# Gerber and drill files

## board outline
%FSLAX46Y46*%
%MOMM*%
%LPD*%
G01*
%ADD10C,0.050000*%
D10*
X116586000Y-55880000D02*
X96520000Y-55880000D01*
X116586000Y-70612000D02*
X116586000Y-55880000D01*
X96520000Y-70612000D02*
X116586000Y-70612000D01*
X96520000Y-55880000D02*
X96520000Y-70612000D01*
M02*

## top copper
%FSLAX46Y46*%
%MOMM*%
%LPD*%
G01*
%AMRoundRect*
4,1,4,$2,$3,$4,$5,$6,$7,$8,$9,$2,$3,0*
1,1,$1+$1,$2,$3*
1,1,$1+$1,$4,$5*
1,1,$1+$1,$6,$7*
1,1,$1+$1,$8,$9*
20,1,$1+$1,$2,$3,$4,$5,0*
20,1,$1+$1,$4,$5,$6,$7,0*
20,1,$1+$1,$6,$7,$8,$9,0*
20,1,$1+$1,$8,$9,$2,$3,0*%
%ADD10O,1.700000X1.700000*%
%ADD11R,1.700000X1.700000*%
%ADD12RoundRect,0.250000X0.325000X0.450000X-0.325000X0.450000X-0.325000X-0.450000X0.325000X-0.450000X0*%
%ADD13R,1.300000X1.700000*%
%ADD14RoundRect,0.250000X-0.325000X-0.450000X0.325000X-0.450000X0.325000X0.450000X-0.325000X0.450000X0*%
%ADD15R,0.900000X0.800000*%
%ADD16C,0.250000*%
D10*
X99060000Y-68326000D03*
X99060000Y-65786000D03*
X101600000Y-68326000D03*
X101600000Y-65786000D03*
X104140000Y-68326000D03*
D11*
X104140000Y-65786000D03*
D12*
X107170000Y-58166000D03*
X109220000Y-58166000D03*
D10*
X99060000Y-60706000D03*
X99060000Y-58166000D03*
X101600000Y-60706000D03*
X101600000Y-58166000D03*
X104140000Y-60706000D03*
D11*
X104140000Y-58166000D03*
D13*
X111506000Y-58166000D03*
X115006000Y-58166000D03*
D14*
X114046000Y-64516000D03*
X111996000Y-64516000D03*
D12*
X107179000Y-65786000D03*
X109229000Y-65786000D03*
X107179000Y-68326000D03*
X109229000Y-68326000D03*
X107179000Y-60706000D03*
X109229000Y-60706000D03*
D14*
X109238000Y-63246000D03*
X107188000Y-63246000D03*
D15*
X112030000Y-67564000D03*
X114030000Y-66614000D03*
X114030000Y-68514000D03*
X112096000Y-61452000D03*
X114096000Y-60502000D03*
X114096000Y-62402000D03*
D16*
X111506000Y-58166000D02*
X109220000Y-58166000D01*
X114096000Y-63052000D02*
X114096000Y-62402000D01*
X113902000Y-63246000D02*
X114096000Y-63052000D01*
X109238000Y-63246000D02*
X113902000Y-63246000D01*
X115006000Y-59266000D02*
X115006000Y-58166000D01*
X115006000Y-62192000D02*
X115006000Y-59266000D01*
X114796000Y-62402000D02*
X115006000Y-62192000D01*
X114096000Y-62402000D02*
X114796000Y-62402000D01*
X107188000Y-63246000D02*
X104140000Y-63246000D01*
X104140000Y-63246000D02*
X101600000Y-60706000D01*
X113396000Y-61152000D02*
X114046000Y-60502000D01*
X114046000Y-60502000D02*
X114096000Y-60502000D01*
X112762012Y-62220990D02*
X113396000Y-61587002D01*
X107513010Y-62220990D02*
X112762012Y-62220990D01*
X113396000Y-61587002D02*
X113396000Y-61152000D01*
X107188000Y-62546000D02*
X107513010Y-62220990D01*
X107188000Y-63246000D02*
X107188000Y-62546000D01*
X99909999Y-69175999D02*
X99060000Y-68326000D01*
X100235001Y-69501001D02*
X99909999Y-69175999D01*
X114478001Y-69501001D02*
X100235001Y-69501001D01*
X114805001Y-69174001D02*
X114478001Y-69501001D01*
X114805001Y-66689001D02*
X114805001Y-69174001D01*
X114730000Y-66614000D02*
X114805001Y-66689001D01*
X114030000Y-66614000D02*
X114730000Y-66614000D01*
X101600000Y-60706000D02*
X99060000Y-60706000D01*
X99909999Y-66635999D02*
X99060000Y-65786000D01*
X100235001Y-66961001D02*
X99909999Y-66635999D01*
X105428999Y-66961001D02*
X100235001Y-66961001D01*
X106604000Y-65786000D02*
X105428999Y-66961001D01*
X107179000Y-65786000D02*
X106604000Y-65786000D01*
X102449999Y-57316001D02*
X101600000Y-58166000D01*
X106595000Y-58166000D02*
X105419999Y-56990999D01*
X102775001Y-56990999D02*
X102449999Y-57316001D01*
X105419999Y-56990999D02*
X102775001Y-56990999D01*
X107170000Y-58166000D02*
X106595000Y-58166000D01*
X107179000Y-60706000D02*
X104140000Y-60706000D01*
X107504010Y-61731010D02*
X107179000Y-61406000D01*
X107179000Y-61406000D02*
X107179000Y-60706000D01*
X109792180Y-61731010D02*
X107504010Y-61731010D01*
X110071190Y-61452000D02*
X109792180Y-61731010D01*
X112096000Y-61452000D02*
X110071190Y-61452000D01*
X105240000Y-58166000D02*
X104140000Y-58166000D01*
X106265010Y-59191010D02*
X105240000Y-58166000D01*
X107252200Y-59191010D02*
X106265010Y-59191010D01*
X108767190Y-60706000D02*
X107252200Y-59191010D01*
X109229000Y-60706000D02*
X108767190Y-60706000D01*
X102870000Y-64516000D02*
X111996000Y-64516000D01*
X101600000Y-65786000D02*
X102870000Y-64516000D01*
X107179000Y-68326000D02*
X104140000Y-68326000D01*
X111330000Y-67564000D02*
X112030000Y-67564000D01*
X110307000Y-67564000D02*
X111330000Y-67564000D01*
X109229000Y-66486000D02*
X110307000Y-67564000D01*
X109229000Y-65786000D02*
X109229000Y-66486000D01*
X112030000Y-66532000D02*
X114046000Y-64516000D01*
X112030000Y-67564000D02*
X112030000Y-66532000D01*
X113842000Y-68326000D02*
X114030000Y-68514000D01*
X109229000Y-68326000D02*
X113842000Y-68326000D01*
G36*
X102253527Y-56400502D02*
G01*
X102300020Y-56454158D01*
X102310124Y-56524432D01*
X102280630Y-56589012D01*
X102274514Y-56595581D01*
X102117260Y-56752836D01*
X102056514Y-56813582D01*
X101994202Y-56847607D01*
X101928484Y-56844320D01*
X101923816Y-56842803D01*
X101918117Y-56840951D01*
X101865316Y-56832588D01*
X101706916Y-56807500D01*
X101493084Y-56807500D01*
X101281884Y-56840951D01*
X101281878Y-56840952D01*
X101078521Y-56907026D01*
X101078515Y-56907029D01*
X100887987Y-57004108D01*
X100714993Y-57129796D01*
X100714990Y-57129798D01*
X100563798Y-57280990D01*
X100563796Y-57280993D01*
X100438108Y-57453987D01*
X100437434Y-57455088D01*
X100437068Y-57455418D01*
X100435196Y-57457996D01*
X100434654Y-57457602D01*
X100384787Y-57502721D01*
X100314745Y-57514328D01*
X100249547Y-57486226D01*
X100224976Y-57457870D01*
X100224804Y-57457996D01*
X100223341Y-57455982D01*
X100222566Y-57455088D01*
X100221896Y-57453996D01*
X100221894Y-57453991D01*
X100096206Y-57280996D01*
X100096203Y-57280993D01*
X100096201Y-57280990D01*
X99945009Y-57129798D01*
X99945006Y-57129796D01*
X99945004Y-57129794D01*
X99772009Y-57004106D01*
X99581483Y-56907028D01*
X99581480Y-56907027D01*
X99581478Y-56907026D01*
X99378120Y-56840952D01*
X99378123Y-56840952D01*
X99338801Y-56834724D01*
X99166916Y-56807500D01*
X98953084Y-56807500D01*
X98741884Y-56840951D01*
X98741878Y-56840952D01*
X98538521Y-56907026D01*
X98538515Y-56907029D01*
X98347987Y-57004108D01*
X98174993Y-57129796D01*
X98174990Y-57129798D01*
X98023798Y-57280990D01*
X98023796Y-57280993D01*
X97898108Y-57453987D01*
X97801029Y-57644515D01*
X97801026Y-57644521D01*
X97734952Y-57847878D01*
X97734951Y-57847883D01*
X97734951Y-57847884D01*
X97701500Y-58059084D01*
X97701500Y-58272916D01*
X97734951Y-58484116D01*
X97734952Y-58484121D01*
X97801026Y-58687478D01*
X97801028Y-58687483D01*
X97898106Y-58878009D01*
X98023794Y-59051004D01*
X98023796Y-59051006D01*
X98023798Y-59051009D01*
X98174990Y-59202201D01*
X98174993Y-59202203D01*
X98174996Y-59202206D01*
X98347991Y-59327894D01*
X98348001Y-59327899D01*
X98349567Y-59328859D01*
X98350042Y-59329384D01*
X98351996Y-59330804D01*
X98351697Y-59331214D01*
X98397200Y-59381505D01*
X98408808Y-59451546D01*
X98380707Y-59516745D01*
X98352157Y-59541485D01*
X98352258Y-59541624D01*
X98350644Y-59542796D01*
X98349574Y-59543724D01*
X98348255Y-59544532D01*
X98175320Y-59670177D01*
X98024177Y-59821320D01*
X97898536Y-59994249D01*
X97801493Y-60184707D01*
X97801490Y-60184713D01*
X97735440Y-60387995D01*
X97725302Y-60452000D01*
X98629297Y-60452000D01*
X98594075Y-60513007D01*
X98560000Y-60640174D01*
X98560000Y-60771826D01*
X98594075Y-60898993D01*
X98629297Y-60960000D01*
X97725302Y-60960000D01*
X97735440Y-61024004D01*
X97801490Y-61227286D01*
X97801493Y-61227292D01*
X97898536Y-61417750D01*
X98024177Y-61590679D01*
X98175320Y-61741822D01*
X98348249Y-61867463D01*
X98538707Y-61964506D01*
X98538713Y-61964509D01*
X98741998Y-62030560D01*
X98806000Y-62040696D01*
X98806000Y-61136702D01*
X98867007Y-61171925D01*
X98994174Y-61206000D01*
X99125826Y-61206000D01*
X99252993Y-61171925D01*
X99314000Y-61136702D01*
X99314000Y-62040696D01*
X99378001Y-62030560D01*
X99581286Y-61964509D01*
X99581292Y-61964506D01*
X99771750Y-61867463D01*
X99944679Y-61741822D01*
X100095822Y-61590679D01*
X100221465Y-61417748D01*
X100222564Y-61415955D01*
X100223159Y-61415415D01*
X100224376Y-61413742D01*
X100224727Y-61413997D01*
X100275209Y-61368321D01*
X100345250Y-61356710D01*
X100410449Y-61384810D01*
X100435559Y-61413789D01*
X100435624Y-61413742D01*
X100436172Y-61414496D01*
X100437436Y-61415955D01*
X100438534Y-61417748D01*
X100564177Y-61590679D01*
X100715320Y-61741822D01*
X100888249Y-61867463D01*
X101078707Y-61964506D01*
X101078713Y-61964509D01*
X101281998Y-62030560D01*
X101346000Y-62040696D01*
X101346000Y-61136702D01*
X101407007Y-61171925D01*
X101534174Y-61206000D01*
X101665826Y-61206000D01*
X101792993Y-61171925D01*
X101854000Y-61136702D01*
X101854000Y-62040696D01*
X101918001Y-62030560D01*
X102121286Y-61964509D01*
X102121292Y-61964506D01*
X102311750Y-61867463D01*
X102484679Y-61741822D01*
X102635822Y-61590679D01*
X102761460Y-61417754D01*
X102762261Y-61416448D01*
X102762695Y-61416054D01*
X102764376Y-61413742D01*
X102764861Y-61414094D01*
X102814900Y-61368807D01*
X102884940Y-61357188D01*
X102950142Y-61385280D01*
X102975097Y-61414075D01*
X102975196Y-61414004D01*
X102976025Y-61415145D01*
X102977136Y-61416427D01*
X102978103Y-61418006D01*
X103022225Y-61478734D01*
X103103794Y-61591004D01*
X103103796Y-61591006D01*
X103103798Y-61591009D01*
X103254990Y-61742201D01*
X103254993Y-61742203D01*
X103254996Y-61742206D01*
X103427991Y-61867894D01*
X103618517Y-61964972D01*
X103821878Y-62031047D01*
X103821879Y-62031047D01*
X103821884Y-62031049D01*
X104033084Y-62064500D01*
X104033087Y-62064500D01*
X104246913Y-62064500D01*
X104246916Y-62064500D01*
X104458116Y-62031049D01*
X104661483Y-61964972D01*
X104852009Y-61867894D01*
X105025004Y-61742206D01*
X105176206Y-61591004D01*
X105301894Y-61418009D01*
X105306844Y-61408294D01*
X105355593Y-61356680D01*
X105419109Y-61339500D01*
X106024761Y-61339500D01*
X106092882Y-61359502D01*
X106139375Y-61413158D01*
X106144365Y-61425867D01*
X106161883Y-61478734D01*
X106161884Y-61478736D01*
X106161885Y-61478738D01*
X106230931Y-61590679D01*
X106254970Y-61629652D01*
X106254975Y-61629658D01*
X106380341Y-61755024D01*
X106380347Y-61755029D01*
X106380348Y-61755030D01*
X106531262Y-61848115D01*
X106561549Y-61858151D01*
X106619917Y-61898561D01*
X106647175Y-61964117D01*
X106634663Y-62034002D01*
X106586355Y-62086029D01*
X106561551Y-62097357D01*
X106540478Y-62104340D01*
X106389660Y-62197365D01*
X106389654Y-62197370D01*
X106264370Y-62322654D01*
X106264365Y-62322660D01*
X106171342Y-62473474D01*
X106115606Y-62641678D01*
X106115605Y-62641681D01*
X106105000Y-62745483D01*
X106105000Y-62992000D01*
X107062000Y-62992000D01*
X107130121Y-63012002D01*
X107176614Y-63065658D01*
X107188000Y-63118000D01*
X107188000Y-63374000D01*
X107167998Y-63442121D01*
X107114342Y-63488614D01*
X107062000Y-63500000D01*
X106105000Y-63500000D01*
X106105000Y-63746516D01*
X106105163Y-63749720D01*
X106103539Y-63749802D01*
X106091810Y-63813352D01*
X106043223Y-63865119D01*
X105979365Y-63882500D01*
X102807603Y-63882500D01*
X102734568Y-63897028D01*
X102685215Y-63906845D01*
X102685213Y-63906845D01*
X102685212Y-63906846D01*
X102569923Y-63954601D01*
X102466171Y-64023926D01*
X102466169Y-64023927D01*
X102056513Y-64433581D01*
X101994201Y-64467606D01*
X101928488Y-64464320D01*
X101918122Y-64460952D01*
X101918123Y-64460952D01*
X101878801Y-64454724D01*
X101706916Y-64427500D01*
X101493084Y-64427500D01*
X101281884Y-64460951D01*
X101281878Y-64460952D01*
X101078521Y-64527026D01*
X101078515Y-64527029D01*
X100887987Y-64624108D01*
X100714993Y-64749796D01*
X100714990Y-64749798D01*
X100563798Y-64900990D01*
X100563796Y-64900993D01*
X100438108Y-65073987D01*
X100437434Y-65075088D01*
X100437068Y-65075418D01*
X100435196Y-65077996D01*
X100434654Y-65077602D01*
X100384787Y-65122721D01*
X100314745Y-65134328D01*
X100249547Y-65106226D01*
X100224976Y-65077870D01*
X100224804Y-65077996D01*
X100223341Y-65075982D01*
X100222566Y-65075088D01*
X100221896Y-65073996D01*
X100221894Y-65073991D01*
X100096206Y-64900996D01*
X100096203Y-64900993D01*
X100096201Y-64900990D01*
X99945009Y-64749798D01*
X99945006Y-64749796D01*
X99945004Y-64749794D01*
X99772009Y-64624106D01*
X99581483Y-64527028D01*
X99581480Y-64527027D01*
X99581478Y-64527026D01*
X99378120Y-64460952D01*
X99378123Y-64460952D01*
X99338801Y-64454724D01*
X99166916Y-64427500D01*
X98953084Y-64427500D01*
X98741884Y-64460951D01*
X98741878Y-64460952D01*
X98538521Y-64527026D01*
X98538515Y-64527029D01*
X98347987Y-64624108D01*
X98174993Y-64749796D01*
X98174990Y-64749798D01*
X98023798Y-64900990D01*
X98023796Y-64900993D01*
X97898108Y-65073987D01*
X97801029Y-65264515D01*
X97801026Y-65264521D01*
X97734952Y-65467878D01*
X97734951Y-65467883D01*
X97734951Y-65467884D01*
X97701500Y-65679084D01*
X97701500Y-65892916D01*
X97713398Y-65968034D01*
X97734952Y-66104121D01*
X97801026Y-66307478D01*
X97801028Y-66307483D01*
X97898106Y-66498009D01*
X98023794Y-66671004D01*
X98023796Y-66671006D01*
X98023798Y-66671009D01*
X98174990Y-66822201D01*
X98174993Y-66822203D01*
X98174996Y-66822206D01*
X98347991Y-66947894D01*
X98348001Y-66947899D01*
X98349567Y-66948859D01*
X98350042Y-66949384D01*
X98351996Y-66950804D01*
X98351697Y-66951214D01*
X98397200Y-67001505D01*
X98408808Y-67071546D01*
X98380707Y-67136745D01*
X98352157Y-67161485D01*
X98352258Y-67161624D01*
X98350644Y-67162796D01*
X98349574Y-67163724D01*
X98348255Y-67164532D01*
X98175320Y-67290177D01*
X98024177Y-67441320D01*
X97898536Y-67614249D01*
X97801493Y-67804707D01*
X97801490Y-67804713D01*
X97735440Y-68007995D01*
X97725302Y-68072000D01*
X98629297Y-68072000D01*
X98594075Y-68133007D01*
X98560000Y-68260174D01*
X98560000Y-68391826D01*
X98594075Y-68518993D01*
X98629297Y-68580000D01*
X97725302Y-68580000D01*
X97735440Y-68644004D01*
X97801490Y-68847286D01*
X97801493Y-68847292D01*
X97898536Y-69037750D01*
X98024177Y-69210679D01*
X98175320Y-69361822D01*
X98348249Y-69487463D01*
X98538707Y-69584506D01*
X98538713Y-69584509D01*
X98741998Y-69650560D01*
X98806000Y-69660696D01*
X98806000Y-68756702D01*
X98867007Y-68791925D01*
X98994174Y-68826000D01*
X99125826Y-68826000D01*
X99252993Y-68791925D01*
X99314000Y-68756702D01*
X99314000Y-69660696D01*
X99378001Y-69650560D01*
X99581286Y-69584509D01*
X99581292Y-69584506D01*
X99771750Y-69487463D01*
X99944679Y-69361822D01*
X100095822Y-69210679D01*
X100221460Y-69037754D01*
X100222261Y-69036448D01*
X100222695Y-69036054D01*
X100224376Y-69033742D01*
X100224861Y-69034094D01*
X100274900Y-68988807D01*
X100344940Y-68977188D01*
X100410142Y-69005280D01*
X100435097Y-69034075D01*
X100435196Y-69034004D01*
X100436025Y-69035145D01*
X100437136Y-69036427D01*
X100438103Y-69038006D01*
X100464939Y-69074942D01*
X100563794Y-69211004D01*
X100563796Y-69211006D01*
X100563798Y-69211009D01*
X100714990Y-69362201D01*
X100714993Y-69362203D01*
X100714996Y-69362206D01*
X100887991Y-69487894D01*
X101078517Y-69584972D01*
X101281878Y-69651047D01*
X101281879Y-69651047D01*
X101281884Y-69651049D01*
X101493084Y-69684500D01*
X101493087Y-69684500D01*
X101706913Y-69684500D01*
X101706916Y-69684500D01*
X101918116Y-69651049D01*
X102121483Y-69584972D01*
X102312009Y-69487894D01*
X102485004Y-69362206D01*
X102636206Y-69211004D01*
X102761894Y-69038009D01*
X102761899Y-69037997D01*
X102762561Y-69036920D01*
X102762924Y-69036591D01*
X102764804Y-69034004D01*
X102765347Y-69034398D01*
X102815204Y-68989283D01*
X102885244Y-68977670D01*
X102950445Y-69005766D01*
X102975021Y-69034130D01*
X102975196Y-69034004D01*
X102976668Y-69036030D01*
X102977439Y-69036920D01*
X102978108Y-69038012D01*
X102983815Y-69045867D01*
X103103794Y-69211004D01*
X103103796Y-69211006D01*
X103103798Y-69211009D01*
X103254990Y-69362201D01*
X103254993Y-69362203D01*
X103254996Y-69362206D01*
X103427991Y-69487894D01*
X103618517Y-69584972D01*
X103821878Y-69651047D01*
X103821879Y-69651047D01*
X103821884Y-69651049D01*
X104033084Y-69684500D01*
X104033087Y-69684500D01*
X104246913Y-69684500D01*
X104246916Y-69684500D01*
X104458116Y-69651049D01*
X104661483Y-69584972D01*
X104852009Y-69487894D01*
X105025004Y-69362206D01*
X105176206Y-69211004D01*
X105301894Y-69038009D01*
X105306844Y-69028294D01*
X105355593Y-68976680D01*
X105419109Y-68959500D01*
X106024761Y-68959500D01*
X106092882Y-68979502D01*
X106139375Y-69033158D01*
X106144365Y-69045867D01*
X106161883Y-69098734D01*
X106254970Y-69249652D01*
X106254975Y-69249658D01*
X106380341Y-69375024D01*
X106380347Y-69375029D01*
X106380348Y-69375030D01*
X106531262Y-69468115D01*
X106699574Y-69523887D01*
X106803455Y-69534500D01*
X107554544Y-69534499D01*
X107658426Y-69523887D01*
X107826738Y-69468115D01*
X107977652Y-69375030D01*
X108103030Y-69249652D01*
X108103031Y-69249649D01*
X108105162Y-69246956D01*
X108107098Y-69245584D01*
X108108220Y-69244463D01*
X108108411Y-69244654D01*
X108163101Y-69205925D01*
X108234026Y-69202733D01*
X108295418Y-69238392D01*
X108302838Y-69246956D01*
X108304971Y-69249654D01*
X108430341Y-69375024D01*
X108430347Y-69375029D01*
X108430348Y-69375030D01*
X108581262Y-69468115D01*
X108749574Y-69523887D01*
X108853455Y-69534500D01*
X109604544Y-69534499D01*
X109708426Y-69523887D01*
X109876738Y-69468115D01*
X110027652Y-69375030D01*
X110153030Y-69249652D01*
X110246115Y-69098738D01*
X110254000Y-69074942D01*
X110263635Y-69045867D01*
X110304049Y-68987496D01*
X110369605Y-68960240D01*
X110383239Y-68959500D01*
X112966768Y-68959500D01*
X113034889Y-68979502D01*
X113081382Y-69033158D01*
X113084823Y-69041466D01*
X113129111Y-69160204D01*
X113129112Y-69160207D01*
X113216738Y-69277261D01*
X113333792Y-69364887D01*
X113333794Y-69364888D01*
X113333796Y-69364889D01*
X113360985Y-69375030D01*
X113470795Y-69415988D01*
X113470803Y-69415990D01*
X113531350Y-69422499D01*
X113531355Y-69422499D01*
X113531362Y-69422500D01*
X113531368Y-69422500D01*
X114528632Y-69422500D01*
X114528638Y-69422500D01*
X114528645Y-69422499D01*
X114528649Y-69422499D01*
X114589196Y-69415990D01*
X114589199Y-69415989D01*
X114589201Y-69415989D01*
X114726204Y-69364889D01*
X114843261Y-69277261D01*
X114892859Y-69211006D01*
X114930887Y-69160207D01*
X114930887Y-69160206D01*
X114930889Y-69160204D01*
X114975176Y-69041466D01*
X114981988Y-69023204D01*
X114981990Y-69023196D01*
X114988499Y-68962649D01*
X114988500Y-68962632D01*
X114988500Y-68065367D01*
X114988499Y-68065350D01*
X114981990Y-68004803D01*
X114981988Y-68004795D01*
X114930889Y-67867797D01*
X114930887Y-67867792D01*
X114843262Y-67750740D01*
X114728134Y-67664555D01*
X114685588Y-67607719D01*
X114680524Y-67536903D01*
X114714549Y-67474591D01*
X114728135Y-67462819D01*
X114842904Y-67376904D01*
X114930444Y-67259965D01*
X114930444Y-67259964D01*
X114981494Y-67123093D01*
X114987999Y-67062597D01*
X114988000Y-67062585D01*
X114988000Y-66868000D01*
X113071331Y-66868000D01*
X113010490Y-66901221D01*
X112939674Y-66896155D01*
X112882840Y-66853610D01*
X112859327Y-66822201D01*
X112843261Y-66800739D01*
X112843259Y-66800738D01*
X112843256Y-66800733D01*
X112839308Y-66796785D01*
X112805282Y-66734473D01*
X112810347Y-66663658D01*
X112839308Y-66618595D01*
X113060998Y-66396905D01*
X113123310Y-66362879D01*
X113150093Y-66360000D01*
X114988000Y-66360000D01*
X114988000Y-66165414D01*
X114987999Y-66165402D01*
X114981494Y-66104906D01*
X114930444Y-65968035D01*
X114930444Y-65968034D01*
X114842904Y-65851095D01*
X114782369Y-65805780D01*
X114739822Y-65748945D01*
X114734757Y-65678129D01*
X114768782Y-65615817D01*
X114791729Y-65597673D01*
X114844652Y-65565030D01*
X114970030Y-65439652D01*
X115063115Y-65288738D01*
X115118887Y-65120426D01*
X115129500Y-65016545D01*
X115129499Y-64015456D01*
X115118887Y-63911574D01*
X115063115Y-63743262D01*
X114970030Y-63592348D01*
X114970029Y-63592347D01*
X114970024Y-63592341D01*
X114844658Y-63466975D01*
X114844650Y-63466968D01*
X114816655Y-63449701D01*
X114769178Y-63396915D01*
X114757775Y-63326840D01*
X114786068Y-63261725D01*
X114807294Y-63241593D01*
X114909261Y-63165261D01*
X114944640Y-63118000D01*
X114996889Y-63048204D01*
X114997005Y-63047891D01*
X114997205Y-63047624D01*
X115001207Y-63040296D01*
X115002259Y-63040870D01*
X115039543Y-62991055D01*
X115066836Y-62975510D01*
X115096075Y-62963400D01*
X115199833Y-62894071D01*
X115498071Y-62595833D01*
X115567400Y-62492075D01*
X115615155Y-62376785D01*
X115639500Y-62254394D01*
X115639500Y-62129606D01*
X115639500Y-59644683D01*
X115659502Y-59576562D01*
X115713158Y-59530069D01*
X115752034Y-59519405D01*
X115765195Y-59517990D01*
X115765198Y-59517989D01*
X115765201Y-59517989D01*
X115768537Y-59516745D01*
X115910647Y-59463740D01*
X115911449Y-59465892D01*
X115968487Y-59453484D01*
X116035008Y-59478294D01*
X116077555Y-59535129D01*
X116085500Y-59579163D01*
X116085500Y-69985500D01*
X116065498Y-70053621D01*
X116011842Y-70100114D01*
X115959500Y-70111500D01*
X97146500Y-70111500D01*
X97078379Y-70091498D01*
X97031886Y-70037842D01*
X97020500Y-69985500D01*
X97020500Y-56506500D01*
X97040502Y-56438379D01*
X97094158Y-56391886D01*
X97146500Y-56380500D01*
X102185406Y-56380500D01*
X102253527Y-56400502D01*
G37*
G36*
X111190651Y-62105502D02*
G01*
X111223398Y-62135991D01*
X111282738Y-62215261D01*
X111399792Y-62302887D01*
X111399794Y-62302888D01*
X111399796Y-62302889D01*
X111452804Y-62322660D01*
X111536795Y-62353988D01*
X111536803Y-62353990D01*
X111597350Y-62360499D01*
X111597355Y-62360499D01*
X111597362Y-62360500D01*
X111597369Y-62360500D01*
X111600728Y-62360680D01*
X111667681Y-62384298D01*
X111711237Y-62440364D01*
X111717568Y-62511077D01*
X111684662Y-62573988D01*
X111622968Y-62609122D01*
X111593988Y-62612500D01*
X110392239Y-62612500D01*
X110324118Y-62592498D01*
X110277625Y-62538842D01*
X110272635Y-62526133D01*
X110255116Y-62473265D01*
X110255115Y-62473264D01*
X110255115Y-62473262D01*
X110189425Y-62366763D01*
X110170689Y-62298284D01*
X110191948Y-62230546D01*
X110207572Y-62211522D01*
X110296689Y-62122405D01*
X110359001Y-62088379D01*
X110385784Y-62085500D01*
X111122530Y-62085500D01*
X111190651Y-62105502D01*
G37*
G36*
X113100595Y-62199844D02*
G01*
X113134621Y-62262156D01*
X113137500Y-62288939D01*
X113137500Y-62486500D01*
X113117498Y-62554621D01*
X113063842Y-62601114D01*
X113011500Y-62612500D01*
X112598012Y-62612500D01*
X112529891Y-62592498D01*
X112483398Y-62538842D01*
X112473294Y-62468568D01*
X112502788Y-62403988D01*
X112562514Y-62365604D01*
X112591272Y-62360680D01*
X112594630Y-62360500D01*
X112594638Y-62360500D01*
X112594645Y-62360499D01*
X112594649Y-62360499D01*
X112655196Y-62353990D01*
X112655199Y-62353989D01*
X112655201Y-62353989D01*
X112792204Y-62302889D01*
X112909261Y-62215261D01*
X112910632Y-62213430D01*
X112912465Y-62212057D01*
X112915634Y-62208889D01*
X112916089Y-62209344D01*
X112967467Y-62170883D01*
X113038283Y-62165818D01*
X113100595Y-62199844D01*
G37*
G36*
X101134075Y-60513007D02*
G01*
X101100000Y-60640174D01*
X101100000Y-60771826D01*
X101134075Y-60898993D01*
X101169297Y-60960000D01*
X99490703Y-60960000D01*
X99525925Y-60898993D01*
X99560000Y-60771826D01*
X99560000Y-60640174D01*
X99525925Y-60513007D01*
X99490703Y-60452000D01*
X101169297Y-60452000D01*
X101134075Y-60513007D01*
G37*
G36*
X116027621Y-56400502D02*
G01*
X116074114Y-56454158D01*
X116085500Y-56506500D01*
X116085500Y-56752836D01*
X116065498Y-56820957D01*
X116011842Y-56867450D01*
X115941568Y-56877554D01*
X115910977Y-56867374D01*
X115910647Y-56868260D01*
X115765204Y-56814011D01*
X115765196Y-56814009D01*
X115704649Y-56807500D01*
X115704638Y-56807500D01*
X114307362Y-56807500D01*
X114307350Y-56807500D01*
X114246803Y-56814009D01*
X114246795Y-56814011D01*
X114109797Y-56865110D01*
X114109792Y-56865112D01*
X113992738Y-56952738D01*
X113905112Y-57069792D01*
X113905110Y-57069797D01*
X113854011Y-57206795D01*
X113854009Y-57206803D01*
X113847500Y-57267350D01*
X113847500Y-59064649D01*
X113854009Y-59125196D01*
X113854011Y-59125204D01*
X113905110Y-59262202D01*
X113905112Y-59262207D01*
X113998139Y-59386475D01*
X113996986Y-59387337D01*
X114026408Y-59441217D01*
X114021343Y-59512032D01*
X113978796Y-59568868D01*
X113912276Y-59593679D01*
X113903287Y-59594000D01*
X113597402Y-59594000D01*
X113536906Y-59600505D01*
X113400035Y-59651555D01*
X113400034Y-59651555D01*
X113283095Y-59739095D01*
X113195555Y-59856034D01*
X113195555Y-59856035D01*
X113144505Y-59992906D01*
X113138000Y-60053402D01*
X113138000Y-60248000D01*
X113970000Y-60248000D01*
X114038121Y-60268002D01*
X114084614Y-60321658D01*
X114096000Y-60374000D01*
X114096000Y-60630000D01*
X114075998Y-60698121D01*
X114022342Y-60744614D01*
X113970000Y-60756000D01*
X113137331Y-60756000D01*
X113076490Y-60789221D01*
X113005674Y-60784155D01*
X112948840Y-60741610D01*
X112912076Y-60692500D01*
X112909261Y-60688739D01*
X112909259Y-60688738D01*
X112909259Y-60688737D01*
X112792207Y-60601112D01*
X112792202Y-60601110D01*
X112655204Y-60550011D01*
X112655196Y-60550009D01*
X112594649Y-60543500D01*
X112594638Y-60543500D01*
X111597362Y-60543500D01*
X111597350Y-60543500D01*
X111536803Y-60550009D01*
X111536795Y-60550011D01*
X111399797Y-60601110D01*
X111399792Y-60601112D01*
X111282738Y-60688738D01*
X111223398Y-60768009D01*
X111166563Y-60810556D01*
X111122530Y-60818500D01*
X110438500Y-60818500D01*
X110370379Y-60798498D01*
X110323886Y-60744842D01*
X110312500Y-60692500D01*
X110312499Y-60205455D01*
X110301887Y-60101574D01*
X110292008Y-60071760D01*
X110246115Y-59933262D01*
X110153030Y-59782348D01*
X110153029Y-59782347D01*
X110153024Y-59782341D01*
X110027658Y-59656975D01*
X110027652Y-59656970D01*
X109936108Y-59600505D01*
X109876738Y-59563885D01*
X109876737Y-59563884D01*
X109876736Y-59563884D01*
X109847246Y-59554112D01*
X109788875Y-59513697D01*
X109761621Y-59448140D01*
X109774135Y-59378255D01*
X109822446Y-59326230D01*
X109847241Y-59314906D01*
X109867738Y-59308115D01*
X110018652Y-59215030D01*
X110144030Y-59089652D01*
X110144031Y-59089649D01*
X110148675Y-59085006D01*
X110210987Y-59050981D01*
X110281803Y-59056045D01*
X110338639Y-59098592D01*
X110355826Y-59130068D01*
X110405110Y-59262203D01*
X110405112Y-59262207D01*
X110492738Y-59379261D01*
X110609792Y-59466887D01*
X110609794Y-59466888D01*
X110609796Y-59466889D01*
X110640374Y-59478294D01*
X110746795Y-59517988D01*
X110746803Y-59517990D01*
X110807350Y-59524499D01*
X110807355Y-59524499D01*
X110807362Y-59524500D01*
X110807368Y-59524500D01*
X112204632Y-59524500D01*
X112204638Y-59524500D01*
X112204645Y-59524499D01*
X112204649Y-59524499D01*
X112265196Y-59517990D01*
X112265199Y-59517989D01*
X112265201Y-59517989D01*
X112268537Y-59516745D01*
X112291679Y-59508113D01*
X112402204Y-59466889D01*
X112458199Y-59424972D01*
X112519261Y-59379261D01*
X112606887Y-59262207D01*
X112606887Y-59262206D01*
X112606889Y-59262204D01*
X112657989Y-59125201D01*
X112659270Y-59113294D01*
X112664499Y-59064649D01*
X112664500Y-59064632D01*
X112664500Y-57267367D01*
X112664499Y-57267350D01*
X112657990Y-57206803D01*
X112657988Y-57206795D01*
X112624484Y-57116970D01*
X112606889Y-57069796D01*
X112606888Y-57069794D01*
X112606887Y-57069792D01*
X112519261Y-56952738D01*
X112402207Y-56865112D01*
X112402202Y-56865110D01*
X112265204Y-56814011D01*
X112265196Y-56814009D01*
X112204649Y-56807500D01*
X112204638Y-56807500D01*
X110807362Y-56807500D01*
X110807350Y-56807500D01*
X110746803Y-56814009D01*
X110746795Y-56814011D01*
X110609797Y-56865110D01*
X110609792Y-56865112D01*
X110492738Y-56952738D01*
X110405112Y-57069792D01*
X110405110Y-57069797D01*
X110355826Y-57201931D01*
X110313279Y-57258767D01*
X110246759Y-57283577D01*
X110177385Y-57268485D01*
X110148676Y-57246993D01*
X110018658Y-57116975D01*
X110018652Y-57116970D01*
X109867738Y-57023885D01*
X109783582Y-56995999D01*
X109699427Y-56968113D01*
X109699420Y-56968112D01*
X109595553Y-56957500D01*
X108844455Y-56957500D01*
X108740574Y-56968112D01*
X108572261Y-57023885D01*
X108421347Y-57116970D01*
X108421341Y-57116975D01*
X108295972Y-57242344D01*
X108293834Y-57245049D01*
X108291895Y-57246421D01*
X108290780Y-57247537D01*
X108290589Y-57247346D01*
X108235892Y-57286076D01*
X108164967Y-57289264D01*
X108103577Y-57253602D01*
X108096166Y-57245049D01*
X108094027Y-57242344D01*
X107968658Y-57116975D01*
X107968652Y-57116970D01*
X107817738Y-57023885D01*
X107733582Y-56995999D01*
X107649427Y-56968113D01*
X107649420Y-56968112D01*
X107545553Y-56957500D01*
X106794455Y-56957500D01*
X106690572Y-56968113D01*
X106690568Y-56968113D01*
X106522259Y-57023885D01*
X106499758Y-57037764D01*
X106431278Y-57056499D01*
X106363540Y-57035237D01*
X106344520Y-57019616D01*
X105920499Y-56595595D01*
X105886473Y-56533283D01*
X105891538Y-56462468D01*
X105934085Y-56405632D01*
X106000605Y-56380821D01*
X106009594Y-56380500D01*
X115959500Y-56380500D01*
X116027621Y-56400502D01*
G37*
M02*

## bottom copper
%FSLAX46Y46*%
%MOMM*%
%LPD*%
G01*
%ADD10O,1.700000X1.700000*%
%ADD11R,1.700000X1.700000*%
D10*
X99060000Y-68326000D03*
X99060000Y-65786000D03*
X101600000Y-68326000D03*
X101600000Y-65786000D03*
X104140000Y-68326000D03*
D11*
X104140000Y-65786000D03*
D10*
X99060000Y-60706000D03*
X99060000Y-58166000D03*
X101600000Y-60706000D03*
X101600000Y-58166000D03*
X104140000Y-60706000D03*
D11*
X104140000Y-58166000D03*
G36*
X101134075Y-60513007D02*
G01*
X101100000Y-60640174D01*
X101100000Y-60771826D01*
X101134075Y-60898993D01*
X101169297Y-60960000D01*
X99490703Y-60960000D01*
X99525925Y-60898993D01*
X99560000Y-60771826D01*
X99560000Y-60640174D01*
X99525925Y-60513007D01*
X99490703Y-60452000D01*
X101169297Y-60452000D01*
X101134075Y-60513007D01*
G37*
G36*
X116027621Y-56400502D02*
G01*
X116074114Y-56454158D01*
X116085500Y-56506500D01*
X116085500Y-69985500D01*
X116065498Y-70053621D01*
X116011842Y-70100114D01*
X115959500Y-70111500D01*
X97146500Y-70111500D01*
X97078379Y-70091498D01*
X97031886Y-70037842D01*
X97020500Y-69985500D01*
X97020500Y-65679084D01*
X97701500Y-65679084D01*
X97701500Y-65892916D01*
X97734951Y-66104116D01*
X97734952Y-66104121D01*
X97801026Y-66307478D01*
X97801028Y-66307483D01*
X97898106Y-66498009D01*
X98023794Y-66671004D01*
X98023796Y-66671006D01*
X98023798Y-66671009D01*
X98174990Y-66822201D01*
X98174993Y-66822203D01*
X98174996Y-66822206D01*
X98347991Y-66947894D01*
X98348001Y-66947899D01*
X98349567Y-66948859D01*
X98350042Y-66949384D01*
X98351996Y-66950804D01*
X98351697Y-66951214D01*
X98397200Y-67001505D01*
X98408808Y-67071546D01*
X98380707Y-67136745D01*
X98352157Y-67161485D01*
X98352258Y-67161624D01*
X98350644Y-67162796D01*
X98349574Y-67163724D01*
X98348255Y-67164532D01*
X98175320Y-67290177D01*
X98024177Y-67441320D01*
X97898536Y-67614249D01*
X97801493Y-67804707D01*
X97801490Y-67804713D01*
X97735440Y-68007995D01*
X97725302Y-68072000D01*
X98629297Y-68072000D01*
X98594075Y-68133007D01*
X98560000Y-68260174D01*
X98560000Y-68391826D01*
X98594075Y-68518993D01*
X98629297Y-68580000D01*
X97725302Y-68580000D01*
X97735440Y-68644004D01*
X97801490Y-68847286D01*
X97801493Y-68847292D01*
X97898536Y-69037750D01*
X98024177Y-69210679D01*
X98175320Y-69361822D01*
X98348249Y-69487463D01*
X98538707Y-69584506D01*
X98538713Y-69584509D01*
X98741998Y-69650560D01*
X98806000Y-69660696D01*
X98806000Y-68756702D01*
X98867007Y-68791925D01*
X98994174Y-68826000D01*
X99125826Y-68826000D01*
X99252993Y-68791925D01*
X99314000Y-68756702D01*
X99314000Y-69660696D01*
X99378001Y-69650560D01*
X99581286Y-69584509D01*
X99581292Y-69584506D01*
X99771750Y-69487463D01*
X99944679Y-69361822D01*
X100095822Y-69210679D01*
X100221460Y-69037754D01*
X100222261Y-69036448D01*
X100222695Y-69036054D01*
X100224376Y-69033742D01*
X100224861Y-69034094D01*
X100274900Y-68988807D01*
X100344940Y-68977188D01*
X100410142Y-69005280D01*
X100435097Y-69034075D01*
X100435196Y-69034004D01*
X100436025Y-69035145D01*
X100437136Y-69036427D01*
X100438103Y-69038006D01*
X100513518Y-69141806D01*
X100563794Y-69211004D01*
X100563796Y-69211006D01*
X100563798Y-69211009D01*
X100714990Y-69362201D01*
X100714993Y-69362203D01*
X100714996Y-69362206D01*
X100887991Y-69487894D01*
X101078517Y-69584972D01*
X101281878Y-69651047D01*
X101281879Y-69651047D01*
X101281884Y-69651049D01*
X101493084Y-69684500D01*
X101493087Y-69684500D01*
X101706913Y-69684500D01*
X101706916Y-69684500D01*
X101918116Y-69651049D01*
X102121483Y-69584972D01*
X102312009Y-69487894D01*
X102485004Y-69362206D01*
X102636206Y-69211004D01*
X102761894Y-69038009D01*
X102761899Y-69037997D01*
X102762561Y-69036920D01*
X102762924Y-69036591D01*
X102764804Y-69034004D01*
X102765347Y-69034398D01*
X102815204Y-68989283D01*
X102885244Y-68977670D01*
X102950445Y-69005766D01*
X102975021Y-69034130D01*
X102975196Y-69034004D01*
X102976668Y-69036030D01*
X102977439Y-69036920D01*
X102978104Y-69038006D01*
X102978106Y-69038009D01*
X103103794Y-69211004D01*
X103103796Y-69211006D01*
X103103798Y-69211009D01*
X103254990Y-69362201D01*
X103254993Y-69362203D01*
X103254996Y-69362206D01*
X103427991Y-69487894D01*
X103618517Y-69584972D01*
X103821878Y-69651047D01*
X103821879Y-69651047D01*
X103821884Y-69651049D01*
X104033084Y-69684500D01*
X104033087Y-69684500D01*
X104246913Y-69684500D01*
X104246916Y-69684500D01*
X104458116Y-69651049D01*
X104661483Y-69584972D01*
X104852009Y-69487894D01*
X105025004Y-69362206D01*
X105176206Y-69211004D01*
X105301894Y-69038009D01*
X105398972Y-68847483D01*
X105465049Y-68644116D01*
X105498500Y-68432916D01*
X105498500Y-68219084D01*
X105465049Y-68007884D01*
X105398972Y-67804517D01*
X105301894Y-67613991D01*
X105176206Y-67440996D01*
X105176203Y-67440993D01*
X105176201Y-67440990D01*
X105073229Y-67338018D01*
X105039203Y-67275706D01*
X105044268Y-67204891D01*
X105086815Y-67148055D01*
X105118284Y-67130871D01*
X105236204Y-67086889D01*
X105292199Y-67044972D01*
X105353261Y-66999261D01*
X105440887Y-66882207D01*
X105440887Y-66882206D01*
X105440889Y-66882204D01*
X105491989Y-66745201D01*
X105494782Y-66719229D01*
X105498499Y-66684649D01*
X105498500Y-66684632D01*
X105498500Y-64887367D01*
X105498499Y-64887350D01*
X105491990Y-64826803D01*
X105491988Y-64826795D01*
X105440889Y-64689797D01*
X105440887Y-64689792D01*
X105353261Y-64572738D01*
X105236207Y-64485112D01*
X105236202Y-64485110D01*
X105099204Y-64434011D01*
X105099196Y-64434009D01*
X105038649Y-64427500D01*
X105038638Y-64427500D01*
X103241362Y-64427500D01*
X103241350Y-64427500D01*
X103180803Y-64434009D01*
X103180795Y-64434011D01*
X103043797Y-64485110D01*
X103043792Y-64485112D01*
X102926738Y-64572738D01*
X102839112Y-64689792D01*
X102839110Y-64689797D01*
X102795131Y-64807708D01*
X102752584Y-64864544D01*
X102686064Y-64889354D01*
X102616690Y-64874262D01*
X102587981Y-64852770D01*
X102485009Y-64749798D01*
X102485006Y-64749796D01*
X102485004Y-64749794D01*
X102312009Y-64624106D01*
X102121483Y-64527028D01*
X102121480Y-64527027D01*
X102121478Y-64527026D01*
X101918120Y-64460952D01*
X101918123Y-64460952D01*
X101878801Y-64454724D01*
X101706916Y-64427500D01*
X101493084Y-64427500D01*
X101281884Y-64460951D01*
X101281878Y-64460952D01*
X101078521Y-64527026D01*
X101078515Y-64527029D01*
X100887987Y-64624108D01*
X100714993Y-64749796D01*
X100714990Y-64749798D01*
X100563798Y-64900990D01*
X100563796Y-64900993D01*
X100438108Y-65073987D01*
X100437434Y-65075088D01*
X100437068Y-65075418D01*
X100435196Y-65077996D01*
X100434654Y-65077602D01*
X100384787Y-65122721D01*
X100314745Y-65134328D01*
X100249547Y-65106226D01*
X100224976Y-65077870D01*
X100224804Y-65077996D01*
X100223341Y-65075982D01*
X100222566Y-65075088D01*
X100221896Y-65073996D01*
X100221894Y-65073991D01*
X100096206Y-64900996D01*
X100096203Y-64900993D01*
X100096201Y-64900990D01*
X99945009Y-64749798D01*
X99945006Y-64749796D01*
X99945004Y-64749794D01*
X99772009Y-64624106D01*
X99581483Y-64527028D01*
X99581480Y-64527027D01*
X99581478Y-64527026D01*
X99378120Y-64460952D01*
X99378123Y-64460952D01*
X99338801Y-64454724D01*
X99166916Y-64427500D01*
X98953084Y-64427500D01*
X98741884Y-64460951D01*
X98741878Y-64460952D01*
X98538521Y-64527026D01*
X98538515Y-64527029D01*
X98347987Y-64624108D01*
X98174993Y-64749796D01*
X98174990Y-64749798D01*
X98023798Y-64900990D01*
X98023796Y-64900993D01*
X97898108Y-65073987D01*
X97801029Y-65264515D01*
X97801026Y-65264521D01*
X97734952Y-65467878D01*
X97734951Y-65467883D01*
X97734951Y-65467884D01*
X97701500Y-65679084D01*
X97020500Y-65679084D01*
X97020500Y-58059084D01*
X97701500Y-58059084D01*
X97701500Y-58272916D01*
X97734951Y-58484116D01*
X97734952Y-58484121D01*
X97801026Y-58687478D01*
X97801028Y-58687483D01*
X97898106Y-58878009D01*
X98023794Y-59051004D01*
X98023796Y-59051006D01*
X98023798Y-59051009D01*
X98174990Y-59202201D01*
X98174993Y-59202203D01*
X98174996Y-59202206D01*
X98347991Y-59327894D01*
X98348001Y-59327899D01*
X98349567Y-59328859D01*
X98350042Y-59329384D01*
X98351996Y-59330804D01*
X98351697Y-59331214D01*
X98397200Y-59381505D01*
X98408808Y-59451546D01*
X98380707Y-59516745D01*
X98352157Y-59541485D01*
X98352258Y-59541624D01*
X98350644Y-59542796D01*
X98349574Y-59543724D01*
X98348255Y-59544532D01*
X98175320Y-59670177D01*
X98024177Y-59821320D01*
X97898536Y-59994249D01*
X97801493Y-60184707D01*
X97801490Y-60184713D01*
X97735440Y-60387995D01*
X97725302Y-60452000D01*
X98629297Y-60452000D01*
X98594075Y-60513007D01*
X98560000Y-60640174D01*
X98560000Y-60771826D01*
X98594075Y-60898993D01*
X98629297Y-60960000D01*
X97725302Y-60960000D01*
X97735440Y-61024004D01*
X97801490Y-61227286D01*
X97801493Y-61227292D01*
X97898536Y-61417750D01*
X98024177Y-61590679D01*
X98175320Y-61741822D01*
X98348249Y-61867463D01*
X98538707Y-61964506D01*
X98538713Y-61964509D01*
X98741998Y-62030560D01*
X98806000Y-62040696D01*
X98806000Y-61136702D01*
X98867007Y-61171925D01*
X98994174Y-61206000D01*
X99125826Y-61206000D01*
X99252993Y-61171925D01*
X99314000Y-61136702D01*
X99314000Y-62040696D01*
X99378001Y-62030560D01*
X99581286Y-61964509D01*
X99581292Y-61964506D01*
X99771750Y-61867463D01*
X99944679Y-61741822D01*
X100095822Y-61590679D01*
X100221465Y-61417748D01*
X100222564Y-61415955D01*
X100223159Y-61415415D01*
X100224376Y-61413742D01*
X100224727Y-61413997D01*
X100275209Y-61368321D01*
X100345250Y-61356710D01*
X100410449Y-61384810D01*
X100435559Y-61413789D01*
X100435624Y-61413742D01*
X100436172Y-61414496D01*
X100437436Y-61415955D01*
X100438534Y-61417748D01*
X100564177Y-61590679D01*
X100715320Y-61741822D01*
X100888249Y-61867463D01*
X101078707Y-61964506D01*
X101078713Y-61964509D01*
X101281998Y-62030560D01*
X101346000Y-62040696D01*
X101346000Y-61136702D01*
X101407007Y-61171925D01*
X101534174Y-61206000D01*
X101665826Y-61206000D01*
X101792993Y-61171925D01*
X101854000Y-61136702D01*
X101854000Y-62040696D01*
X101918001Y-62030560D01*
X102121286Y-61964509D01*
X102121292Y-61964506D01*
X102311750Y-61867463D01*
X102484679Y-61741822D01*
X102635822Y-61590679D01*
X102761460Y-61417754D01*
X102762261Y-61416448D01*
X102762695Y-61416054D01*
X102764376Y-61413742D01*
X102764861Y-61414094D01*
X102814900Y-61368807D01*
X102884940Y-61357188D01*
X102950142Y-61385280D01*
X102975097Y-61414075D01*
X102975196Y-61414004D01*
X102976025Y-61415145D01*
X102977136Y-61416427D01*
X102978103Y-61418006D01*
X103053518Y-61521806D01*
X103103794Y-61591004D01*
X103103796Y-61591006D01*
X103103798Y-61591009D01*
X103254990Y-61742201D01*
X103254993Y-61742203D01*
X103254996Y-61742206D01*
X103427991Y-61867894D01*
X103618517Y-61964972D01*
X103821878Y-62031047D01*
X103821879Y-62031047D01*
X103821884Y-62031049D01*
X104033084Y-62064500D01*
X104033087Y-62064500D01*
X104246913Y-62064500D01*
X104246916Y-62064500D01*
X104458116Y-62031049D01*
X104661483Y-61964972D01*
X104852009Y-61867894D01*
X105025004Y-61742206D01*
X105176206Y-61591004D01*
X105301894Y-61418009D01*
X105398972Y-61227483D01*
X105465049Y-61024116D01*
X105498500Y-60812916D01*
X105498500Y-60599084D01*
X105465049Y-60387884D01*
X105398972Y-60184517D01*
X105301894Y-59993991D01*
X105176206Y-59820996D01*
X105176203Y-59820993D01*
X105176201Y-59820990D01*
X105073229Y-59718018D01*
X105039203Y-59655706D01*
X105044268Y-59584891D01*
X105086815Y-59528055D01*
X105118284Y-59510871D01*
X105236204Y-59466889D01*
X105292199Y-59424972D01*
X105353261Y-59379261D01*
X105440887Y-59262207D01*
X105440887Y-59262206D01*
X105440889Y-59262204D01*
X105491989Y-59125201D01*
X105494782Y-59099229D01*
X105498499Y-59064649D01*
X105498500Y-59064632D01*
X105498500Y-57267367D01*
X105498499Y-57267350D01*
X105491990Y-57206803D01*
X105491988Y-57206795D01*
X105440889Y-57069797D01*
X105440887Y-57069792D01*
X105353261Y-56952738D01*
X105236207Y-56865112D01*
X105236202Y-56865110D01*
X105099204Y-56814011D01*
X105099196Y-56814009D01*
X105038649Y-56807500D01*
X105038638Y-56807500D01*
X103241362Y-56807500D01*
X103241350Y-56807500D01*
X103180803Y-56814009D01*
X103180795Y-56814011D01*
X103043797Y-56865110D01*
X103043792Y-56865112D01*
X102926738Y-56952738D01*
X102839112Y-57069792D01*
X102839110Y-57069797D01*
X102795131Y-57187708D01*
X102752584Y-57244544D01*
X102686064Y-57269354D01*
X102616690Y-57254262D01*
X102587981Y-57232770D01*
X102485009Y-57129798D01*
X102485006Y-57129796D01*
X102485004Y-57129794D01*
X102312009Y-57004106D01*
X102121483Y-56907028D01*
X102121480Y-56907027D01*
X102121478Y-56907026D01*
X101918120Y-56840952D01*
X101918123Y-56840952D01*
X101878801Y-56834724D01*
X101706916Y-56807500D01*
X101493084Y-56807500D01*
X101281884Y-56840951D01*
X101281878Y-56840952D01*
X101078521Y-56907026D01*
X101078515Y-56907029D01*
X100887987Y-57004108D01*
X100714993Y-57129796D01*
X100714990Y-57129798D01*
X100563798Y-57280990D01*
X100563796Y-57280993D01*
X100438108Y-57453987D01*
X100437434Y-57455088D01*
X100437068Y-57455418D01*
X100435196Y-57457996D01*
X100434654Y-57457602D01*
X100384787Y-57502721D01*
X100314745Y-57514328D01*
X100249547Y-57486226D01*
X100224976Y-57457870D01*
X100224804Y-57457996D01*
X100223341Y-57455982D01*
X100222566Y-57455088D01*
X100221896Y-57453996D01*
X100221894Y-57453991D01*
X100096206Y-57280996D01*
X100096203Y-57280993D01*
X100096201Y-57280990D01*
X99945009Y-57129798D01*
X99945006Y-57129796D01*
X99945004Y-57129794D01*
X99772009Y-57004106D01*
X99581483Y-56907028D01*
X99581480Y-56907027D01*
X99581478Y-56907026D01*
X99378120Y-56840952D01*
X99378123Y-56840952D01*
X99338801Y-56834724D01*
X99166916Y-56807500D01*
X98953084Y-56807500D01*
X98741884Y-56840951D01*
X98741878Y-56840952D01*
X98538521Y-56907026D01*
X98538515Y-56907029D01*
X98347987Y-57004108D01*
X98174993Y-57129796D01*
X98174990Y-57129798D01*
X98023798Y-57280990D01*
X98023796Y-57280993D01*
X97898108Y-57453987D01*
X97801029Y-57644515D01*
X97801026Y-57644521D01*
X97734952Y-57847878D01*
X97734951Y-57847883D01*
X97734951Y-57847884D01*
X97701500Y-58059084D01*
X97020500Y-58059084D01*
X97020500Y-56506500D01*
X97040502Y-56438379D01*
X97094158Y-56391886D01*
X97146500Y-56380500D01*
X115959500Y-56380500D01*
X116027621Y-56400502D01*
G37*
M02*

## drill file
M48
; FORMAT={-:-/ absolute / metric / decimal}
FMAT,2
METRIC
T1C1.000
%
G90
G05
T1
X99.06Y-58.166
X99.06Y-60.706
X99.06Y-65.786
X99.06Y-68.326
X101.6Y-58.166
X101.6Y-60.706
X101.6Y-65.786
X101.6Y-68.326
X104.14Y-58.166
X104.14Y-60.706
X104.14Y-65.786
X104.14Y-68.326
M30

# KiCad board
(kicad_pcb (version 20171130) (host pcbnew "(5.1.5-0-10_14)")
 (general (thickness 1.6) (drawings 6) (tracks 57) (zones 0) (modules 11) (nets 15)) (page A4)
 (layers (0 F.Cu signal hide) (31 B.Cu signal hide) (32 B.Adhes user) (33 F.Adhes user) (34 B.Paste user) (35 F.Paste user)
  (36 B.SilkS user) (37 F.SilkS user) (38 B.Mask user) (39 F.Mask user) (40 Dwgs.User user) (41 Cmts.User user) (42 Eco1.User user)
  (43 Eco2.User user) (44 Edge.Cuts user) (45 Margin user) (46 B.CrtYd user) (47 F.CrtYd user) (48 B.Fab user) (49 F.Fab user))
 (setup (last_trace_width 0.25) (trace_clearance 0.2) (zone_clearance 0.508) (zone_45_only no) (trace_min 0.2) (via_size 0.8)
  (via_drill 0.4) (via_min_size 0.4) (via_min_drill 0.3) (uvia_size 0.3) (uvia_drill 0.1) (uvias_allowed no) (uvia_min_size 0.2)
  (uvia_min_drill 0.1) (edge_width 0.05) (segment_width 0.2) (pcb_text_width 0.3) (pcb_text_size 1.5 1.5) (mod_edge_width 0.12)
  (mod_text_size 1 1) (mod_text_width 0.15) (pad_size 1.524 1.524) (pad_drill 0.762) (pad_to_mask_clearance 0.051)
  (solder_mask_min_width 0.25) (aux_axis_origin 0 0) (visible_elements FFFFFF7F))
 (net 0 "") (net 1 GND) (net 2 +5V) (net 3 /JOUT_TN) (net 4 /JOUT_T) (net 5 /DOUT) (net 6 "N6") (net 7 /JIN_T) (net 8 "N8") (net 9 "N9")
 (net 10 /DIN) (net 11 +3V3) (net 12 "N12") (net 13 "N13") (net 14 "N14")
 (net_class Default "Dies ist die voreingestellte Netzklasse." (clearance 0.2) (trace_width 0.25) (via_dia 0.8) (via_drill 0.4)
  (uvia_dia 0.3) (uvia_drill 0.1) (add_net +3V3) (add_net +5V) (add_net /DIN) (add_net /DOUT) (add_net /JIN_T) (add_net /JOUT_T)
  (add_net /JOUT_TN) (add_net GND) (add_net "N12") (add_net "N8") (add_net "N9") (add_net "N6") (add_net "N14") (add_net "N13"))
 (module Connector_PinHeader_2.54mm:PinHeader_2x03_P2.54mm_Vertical (layer F.Cu) (at 104.14 65.786 270)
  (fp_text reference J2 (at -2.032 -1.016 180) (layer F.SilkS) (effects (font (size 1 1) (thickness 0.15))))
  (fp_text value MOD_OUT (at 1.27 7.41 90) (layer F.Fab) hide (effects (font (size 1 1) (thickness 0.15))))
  (pad 6 thru_hole oval (at 2.54 5.08 270) (size 1.7 1.7) (drill 1) (layers *.Cu *.Mask) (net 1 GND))
  (pad 5 thru_hole oval (at 0 5.08 270) (size 1.7 1.7) (drill 1) (layers *.Cu *.Mask) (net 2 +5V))
  (pad 4 thru_hole oval (at 2.54 2.54 270) (size 1.7 1.7) (drill 1) (layers *.Cu *.Mask) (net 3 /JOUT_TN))
  (pad 3 thru_hole oval (at 0 2.54 270) (size 1.7 1.7) (drill 1) (layers *.Cu *.Mask) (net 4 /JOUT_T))
  (pad 2 thru_hole oval (at 2.54 0 270) (size 1.7 1.7) (drill 1) (layers *.Cu *.Mask) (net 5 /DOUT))
  (pad 1 thru_hole rect (at 0 0 270) (size 1.7 1.7) (drill 1) (layers *.Cu *.Mask) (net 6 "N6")))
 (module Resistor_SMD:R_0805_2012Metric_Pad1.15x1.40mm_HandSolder (layer F.Cu) (at 108.195 58.166 180)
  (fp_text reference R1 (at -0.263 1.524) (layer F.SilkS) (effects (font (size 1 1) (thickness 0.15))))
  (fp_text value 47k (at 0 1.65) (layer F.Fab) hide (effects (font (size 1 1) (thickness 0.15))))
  (pad 2 smd roundrect (at 1.025 0 180) (size 1.15 1.4) (layers F.Cu F.Paste F.Mask) (roundrect_rratio 0.217391) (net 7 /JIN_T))
  (pad 1 smd roundrect (at -1.025 0 180) (size 1.15 1.4) (layers F.Cu F.Paste F.Mask) (roundrect_rratio 0.217391) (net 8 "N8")))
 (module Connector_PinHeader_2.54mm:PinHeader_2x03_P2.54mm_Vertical (layer F.Cu) (at 104.14 58.166 270)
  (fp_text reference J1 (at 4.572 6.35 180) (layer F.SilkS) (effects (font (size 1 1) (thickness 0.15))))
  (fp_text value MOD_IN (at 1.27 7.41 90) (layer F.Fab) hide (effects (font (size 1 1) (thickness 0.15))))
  (pad 6 thru_hole oval (at 2.54 5.08 270) (size 1.7 1.7) (drill 1) (layers *.Cu *.Mask) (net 1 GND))
  (pad 5 thru_hole oval (at 0 5.08 270) (size 1.7 1.7) (drill 1) (layers *.Cu *.Mask) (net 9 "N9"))
  (pad 4 thru_hole oval (at 2.54 2.54 270) (size 1.7 1.7) (drill 1) (layers *.Cu *.Mask) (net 1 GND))
  (pad 3 thru_hole oval (at 0 2.54 270) (size 1.7 1.7) (drill 1) (layers *.Cu *.Mask) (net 7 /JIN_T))
  (pad 2 thru_hole oval (at 2.54 0 270) (size 1.7 1.7) (drill 1) (layers *.Cu *.Mask) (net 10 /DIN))
  (pad 1 thru_hole rect (at 0 0 270) (size 1.7 1.7) (drill 1) (layers *.Cu *.Mask) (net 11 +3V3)))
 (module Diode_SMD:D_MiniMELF (layer F.Cu) (at 113.256 58.166 180)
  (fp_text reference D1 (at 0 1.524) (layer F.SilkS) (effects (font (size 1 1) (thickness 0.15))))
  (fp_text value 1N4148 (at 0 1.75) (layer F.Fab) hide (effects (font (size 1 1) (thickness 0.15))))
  (pad 2 smd rect (at 1.75 0 180) (size 1.3 1.7) (layers F.Cu F.Paste F.Mask) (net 8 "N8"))
  (pad 1 smd rect (at -1.75 0 180) (size 1.3 1.7) (layers F.Cu F.Paste F.Mask) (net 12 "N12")))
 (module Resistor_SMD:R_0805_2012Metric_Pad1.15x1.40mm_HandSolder (layer F.Cu) (at 113.021 64.516)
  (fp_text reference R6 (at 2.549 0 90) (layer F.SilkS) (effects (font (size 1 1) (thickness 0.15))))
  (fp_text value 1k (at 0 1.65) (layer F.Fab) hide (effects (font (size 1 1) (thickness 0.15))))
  (pad 2 smd roundrect (at 1.025 0) (size 1.15 1.4) (layers F.Cu F.Paste F.Mask) (roundrect_rratio 0.217391) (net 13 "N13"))
  (pad 1 smd roundrect (at -1.025 0) (size 1.15 1.4) (layers F.Cu F.Paste F.Mask) (roundrect_rratio 0.217391) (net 4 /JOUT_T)))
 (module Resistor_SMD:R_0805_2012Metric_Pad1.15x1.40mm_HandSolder (layer F.Cu) (at 108.204 65.786 180)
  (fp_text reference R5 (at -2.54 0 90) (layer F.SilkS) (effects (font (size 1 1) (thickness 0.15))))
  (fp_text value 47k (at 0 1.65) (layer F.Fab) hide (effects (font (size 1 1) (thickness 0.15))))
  (pad 2 smd roundrect (at 1.025 0 180) (size 1.15 1.4) (layers F.Cu F.Paste F.Mask) (roundrect_rratio 0.217391) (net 2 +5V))
  (pad 1 smd roundrect (at -1.025 0 180) (size 1.15 1.4) (layers F.Cu F.Paste F.Mask) (roundrect_rratio 0.217391) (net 13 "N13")))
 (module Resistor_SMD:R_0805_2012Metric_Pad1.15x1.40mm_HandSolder (layer F.Cu) (at 108.204 68.326 180)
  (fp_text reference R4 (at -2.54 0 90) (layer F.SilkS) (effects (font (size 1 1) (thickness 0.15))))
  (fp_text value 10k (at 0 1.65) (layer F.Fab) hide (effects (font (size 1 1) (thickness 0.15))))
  (pad 2 smd roundrect (at 1.025 0 180) (size 1.15 1.4) (layers F.Cu F.Paste F.Mask) (roundrect_rratio 0.217391) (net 5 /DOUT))
  (pad 1 smd roundrect (at -1.025 0 180) (size 1.15 1.4) (layers F.Cu F.Paste F.Mask) (roundrect_rratio 0.217391) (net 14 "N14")))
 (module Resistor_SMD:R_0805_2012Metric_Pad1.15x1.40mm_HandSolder (layer F.Cu) (at 108.204 60.706 180)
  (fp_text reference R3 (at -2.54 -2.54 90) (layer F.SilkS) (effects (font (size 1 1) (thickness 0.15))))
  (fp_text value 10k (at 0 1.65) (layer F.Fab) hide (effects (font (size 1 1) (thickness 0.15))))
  (pad 2 smd roundrect (at 1.025 0 180) (size 1.15 1.4) (layers F.Cu F.Paste F.Mask) (roundrect_rratio 0.217391) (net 10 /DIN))
  (pad 1 smd roundrect (at -1.025 0 180) (size 1.15 1.4) (layers F.Cu F.Paste F.Mask) (roundrect_rratio 0.217391) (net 11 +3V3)))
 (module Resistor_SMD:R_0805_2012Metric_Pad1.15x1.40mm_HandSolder (layer F.Cu) (at 108.213 63.246)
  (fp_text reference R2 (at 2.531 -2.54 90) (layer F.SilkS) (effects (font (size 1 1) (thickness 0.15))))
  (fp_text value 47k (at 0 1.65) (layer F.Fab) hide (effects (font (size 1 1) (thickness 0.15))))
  (pad 2 smd roundrect (at 1.025 0) (size 1.15 1.4) (layers F.Cu F.Paste F.Mask) (roundrect_rratio 0.217391) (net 12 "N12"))
  (pad 1 smd roundrect (at -1.025 0) (size 1.15 1.4) (layers F.Cu F.Paste F.Mask) (roundrect_rratio 0.217391) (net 1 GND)))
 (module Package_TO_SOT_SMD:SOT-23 (layer F.Cu) (at 113.03 67.564 180)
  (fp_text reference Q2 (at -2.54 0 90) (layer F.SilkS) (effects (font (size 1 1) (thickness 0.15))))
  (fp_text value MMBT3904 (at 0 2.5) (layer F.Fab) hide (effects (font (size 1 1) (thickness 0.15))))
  (pad 3 smd rect (at 1 0 180) (size 0.9 0.8) (layers F.Cu F.Paste F.Mask) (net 13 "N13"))
  (pad 2 smd rect (at -1 0.95 180) (size 0.9 0.8) (layers F.Cu F.Paste F.Mask) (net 1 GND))
  (pad 1 smd rect (at -1 -0.95 180) (size 0.9 0.8) (layers F.Cu F.Paste F.Mask) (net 14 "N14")))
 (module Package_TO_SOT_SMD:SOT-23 (layer F.Cu) (at 113.096 61.452 180)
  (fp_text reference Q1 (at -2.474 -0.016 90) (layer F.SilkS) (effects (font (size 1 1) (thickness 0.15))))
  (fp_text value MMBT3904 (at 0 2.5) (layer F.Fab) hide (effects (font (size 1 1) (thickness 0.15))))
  (pad 3 smd rect (at 1 0 180) (size 0.9 0.8) (layers F.Cu F.Paste F.Mask) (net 10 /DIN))
  (pad 2 smd rect (at -1 0.95 180) (size 0.9 0.8) (layers F.Cu F.Paste F.Mask) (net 1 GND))
  (pad 1 smd rect (at -1 -0.95 180) (size 0.9 0.8) (layers F.Cu F.Paste F.Mask) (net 12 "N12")))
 (gr_line (start 116.586 55.88) (end 96.52 55.88) (layer Edge.Cuts) (width 0.05))
 (gr_line (start 116.586 70.612) (end 116.586 55.88) (layer Edge.Cuts) (width 0.05))
 (gr_line (start 96.52 70.612) (end 116.586 70.612) (layer Edge.Cuts) (width 0.05))
 (gr_line (start 96.52 55.88) (end 96.52 70.612) (layer Edge.Cuts) (width 0.05))
 (segment (start 111.506 58.166) (end 109.22 58.166) (width 0.25) (layer F.Cu) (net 8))
 (segment (start 114.096 63.052) (end 114.096 62.402) (width 0.25) (layer F.Cu) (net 12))
 (segment (start 113.902 63.246) (end 114.096 63.052) (width 0.25) (layer F.Cu) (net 12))
 (segment (start 109.238 63.246) (end 113.902 63.246) (width 0.25) (layer F.Cu) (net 12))
 (segment (start 115.006 59.266) (end 115.006 58.166) (width 0.25) (layer F.Cu) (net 12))
 (segment (start 115.006 62.192) (end 115.006 59.266) (width 0.25) (layer F.Cu) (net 12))
 (segment (start 114.796 62.402) (end 115.006 62.192) (width 0.25) (layer F.Cu) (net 12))
 (segment (start 114.096 62.402) (end 114.796 62.402) (width 0.25) (layer F.Cu) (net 12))
 (segment (start 107.188 63.246) (end 104.14 63.246) (width 0.25) (layer F.Cu) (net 1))
 (segment (start 104.14 63.246) (end 101.6 60.706) (width 0.25) (layer F.Cu) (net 1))
 (segment (start 113.396 61.152) (end 114.046 60.502) (width 0.25) (layer F.Cu) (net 1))
 (segment (start 114.046 60.502) (end 114.096 60.502) (width 0.25) (layer F.Cu) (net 1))
 (segment (start 112.762012 62.22099) (end 113.396 61.587002) (width 0.25) (layer F.Cu) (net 1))
 (segment (start 107.51301 62.22099) (end 112.762012 62.22099) (width 0.25) (layer F.Cu) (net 1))
 (segment (start 113.396 61.587002) (end 113.396 61.152) (width 0.25) (layer F.Cu) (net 1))
 (segment (start 107.188 62.546) (end 107.51301 62.22099) (width 0.25) (layer F.Cu) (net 1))
 (segment (start 107.188 63.246) (end 107.188 62.546) (width 0.25) (layer F.Cu) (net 1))
 (segment (start 99.909999 69.175999) (end 99.06 68.326) (width 0.25) (layer F.Cu) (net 1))
 (segment (start 100.235001 69.501001) (end 99.909999 69.175999) (width 0.25) (layer F.Cu) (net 1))
 (segment (start 114.478001 69.501001) (end 100.235001 69.501001) (width 0.25) (layer F.Cu) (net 1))
 (segment (start 114.805001 69.174001) (end 114.478001 69.501001) (width 0.25) (layer F.Cu) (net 1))
 (segment (start 114.805001 66.689001) (end 114.805001 69.174001) (width 0.25) (layer F.Cu) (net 1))
 (segment (start 114.73 66.614) (end 114.805001 66.689001) (width 0.25) (layer F.Cu) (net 1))
 (segment (start 114.03 66.614) (end 114.73 66.614) (width 0.25) (layer F.Cu) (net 1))
 (segment (start 101.6 60.706) (end 99.06 60.706) (width 0.25) (layer F.Cu) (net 1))
 (segment (start 99.909999 66.635999) (end 99.06 65.786) (width 0.25) (layer F.Cu) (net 2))
 (segment (start 100.235001 66.961001) (end 99.909999 66.635999) (width 0.25) (layer F.Cu) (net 2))
 (segment (start 105.428999 66.961001) (end 100.235001 66.961001) (width 0.25) (layer F.Cu) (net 2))
 (segment (start 106.604 65.786) (end 105.428999 66.961001) (width 0.25) (layer F.Cu) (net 2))
 (segment (start 107.179 65.786) (end 106.604 65.786) (width 0.25) (layer F.Cu) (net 2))
 (segment (start 102.449999 57.316001) (end 101.6 58.166) (width 0.25) (layer F.Cu) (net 7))
 (segment (start 106.595 58.166) (end 105.419999 56.990999) (width 0.25) (layer F.Cu) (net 7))
 (segment (start 102.775001 56.990999) (end 102.449999 57.316001) (width 0.25) (layer F.Cu) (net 7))
 (segment (start 105.419999 56.990999) (end 102.775001 56.990999) (width 0.25) (layer F.Cu) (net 7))
 (segment (start 107.17 58.166) (end 106.595 58.166) (width 0.25) (layer F.Cu) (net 7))
 (segment (start 107.179 60.706) (end 104.14 60.706) (width 0.25) (layer F.Cu) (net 10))
 (segment (start 107.50401 61.73101) (end 107.179 61.406) (width 0.25) (layer F.Cu) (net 10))
 (segment (start 107.179 61.406) (end 107.179 60.706) (width 0.25) (layer F.Cu) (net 10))
 (segment (start 109.79218 61.73101) (end 107.50401 61.73101) (width 0.25) (layer F.Cu) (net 10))
 (segment (start 110.07119 61.452) (end 109.79218 61.73101) (width 0.25) (layer F.Cu) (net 10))
 (segment (start 112.096 61.452) (end 110.07119 61.452) (width 0.25) (layer F.Cu) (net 10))
 (segment (start 105.24 58.166) (end 104.14 58.166) (width 0.25) (layer F.Cu) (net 11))
 (segment (start 106.26501 59.19101) (end 105.24 58.166) (width 0.25) (layer F.Cu) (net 11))
 (segment (start 107.2522 59.19101) (end 106.26501 59.19101) (width 0.25) (layer F.Cu) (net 11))
 (segment (start 108.76719 60.706) (end 107.2522 59.19101) (width 0.25) (layer F.Cu) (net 11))
 (segment (start 109.229 60.706) (end 108.76719 60.706) (width 0.25) (layer F.Cu) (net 11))
 (segment (start 102.87 64.516) (end 111.996 64.516) (width 0.25) (layer F.Cu) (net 4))
 (segment (start 101.6 65.786) (end 102.87 64.516) (width 0.25) (layer F.Cu) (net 4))
 (segment (start 107.179 68.326) (end 104.14 68.326) (width 0.25) (layer F.Cu) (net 5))
 (segment (start 111.33 67.564) (end 112.03 67.564) (width 0.25) (layer F.Cu) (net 13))
 (segment (start 110.307 67.564) (end 111.33 67.564) (width 0.25) (layer F.Cu) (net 13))
 (segment (start 109.229 66.486) (end 110.307 67.564) (width 0.25) (layer F.Cu) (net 13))
 (segment (start 109.229 65.786) (end 109.229 66.486) (width 0.25) (layer F.Cu) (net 13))
 (segment (start 112.03 66.532) (end 114.046 64.516) (width 0.25) (layer F.Cu) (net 13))
 (segment (start 112.03 67.564) (end 112.03 66.532) (width 0.25) (layer F.Cu) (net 13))
 (segment (start 113.842 68.326) (end 114.03 68.514) (width 0.25) (layer F.Cu) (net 14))
 (segment (start 109.229 68.326) (end 113.842 68.326) (width 0.25) (layer F.Cu) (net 14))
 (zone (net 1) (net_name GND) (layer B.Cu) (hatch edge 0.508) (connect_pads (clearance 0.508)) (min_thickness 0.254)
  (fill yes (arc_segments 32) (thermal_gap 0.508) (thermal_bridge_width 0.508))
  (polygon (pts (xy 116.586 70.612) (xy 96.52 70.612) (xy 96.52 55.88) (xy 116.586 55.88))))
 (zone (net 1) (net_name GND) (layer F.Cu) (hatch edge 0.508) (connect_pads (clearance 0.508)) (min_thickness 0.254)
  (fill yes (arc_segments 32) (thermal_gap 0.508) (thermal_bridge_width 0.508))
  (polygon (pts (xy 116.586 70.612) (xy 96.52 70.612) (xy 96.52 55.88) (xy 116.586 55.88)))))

